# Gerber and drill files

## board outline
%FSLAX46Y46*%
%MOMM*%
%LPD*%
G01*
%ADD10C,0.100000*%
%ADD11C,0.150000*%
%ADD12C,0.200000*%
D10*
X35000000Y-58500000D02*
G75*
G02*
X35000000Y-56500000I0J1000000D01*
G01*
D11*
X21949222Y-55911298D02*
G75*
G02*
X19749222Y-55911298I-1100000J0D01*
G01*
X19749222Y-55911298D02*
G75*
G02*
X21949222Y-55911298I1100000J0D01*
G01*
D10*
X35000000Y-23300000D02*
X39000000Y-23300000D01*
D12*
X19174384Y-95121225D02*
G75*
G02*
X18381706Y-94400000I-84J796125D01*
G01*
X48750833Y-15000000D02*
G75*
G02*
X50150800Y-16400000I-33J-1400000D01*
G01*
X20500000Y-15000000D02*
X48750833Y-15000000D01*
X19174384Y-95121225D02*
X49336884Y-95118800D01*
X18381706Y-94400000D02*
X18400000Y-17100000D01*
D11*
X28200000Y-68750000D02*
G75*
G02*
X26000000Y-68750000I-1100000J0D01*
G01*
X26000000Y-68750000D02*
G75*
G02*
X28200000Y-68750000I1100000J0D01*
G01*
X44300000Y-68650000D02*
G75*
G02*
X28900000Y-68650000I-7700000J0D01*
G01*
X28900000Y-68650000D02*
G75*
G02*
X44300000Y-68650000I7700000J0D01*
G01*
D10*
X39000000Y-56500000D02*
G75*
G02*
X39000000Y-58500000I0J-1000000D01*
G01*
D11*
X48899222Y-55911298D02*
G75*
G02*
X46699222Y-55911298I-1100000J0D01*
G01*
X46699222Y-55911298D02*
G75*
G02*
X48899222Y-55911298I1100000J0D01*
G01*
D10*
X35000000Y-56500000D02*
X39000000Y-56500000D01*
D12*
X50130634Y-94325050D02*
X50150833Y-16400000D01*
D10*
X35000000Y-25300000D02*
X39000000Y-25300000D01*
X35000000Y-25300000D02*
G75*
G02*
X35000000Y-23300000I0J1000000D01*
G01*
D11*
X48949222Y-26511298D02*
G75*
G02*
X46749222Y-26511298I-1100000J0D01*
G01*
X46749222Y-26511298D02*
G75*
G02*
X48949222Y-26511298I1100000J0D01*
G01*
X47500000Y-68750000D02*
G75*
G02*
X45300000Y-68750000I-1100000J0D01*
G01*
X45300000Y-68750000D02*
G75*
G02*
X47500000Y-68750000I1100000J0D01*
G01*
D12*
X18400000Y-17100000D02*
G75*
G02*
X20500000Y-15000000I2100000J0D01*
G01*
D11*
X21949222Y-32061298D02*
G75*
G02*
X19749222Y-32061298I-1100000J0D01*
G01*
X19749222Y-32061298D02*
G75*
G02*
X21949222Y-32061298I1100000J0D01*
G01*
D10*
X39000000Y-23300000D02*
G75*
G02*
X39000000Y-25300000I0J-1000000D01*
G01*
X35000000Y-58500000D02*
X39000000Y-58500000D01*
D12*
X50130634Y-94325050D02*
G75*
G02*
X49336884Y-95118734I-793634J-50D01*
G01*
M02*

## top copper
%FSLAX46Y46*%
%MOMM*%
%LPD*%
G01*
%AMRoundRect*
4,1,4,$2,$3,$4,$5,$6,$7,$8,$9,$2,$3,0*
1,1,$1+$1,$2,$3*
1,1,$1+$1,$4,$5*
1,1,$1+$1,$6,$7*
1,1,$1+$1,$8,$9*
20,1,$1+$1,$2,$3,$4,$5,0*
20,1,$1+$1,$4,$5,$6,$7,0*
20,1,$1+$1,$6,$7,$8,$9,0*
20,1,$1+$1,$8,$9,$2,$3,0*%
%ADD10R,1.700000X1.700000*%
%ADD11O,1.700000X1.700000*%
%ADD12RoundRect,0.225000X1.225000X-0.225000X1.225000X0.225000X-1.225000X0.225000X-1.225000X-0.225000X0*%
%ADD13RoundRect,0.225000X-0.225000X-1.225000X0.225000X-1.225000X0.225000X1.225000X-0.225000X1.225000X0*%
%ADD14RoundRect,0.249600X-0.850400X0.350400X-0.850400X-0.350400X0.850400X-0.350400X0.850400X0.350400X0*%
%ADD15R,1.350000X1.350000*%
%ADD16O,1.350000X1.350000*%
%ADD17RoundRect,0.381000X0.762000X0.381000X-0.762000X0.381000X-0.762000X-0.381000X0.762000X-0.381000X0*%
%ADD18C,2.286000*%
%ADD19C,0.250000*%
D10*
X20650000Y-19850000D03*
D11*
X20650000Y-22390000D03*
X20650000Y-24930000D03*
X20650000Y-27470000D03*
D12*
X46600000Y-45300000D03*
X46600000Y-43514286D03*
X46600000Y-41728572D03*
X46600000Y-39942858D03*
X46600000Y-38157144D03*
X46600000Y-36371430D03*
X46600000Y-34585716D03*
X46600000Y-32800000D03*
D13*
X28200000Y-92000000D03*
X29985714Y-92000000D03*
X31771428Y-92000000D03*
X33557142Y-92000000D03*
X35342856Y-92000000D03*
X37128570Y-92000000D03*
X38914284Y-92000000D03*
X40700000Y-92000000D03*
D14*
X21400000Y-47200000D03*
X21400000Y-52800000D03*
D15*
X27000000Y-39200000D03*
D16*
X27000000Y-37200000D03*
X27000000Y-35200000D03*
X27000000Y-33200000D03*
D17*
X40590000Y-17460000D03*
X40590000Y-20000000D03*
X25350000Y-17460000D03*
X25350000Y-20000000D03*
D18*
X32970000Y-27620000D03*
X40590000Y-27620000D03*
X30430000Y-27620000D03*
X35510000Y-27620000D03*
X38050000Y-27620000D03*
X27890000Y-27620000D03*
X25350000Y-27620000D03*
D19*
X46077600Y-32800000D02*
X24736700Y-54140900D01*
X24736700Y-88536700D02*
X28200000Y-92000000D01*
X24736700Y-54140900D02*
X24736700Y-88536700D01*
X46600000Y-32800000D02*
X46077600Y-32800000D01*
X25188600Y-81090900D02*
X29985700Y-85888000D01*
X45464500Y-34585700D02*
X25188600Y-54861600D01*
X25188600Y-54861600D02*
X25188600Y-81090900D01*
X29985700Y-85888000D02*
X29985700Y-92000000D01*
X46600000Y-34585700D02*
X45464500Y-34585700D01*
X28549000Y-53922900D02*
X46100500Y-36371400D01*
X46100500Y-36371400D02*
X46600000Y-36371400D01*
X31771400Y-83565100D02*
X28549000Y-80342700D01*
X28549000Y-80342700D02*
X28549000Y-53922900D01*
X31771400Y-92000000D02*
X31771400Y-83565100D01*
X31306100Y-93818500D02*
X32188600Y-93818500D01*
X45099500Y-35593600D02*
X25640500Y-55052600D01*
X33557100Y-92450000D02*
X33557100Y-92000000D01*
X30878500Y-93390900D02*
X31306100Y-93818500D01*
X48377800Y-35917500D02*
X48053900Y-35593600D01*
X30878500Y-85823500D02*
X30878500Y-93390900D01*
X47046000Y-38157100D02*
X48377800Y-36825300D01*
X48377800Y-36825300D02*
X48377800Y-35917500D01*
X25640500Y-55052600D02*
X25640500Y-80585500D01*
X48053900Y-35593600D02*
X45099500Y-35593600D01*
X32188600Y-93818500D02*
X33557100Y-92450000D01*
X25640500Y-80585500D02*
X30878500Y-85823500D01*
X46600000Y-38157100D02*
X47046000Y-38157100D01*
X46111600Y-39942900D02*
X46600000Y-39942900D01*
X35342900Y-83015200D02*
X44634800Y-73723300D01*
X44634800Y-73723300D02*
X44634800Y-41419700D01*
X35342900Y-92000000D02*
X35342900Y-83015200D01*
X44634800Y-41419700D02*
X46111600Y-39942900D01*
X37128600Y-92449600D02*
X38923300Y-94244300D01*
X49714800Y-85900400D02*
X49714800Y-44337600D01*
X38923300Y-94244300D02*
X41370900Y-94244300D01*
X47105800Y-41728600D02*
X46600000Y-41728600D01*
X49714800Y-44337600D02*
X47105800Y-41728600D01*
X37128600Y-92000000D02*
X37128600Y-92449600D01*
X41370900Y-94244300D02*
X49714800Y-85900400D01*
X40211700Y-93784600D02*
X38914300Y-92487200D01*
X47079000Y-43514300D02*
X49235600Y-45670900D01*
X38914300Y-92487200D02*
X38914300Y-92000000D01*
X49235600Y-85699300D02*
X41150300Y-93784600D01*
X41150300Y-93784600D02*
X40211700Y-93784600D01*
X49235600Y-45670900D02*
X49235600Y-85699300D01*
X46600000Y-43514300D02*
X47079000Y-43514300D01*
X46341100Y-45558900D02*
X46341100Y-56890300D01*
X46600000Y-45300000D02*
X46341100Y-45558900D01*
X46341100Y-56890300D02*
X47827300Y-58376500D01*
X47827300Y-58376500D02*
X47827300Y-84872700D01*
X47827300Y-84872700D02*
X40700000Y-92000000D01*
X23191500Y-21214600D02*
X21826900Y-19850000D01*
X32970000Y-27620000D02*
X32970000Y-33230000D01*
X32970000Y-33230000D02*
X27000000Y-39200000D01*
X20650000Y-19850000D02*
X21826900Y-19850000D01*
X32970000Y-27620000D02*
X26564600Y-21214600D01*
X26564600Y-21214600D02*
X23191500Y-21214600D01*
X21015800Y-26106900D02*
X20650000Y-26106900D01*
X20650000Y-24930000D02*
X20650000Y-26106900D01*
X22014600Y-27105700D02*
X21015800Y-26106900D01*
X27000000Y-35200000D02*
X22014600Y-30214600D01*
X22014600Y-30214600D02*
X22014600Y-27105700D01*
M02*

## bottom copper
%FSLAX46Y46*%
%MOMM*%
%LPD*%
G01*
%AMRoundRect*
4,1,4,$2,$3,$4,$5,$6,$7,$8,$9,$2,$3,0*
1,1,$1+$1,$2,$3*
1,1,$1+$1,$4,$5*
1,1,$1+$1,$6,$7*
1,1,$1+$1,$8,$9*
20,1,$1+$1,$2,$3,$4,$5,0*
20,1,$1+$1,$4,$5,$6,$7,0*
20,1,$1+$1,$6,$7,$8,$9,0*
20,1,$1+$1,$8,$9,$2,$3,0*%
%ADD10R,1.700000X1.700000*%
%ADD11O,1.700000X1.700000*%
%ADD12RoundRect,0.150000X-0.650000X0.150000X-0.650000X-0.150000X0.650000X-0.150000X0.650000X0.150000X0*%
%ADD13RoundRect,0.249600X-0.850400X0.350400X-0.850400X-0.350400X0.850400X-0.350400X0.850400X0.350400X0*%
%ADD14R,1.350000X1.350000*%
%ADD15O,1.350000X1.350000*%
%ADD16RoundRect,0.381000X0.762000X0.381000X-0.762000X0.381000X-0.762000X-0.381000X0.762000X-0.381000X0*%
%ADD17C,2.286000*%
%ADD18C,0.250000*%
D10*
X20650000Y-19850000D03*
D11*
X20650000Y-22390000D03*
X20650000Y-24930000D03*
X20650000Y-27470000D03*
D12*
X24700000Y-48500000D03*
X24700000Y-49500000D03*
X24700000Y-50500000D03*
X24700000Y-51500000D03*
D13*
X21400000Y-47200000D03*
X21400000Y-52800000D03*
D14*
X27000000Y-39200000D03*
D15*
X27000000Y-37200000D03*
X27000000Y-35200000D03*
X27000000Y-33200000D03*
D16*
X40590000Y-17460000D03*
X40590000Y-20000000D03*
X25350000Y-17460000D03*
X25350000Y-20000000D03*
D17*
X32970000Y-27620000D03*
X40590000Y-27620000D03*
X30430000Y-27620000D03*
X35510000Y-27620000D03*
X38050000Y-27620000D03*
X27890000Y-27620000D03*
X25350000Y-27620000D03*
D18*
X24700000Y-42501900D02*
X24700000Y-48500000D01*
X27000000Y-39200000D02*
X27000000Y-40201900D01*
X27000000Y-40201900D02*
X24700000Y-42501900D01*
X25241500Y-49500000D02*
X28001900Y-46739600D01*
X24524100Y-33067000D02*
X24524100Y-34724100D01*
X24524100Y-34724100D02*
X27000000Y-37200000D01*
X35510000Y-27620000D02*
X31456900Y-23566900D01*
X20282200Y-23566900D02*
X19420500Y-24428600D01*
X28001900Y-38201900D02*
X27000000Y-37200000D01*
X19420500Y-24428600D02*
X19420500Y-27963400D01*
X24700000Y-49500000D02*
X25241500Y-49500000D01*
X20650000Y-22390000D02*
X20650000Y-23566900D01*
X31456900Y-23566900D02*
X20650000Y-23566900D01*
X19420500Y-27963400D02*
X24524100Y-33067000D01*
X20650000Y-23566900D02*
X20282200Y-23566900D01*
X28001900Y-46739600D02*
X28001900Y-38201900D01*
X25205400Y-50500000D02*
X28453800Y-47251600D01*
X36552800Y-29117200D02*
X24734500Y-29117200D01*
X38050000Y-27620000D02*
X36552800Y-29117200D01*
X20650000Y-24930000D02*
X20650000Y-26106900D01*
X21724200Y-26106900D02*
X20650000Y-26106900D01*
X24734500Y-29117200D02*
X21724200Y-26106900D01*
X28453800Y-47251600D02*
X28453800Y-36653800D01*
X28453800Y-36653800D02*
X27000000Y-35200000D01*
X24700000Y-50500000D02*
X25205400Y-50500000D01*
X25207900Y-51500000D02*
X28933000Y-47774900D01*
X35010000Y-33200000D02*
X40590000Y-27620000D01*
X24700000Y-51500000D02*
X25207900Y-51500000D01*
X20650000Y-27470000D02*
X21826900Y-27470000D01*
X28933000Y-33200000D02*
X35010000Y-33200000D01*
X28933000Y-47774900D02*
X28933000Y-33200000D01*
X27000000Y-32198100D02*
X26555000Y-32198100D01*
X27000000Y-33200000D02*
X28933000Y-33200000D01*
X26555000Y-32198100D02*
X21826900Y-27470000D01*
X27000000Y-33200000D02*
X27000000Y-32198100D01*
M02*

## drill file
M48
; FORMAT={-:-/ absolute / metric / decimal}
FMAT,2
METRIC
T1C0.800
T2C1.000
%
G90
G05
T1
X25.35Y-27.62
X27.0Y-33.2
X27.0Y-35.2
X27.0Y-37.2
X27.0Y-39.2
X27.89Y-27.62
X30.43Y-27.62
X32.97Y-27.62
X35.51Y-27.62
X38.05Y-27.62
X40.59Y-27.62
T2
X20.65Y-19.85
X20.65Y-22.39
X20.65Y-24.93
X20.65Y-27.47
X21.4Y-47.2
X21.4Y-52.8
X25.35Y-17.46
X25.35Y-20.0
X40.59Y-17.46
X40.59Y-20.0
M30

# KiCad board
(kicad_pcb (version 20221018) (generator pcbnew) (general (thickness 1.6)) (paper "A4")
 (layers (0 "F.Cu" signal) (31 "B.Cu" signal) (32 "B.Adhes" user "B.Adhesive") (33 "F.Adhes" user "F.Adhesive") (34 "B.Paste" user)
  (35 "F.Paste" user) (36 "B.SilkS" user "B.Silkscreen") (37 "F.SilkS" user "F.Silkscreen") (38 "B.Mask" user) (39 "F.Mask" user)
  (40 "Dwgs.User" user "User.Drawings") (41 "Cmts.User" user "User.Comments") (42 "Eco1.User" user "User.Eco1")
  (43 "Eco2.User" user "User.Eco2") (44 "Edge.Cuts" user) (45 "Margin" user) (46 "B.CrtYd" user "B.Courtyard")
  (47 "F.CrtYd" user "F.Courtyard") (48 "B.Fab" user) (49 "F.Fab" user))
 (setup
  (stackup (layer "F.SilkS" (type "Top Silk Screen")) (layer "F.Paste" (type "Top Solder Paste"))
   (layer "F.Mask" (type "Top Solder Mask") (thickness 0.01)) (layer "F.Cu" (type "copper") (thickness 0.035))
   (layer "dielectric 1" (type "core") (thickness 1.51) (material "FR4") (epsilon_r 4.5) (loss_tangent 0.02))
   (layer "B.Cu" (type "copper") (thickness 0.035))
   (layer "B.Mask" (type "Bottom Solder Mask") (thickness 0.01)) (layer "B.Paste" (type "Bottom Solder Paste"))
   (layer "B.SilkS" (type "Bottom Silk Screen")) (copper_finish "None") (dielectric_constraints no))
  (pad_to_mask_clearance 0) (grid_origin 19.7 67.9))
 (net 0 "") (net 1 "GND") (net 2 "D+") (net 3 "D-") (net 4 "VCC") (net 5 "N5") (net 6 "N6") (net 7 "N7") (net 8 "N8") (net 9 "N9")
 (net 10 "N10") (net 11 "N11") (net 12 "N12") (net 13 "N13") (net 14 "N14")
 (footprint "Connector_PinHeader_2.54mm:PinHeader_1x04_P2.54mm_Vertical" (layer "F.Cu") (at 20.65 19.85)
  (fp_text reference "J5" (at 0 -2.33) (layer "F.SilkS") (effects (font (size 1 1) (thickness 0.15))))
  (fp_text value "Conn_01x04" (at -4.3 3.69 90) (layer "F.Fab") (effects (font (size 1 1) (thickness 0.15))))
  (pad "1" thru_hole rect (at 0 0) (size 1.7 1.7) (drill 1) (layers "*.Cu" "*.Mask") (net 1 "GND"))
  (pad "2" thru_hole oval (at 0 2.54) (size 1.7 1.7) (drill 1) (layers "*.Cu" "*.Mask") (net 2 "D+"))
  (pad "3" thru_hole oval (at 0 5.08) (size 1.7 1.7) (drill 1) (layers "*.Cu" "*.Mask") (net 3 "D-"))
  (pad "4" thru_hole oval (at 0 7.62) (size 1.7 1.7) (drill 1) (layers "*.Cu" "*.Mask") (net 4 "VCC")))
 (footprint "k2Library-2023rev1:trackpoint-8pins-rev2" (layer "F.Cu") (at 44.1 38.55 90)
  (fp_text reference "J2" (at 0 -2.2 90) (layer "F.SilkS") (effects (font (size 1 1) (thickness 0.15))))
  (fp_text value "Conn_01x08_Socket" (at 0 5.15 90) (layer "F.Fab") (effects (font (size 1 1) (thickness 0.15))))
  (pad "1" smd roundrect (at -6.75 2.5 90) (size 0.9 2.9) (layers "F.Cu" "F.Paste" "F.Mask") (roundrect_rratio 0.25) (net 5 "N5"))
  (pad "2" smd roundrect (at -4.964286 2.5 90) (size 0.9 2.9) (layers "F.Cu" "F.Paste" "F.Mask") (roundrect_rratio 0.25) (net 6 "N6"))
  (pad "3" smd roundrect (at -3.178572 2.5 90) (size 0.9 2.9) (layers "F.Cu" "F.Paste" "F.Mask") (roundrect_rratio 0.25) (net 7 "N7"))
  (pad "4" smd roundrect (at -1.392858 2.5 90) (size 0.9 2.9) (layers "F.Cu" "F.Paste" "F.Mask") (roundrect_rratio 0.25) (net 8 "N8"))
  (pad "5" smd roundrect (at 0.392856 2.5 90) (size 0.9 2.9) (layers "F.Cu" "F.Paste" "F.Mask") (roundrect_rratio 0.25) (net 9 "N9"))
  (pad "6" smd roundrect (at 2.17857 2.5 90) (size 0.9 2.9) (layers "F.Cu" "F.Paste" "F.Mask") (roundrect_rratio 0.25) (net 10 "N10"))
  (pad "7" smd roundrect (at 3.964284 2.5 90) (size 0.9 2.9) (layers "F.Cu" "F.Paste" "F.Mask") (roundrect_rratio 0.25) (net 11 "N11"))
  (pad "8" smd roundrect (at 5.75 2.5 90) (size 0.9 2.9) (layers "F.Cu" "F.Paste" "F.Mask") (roundrect_rratio 0.25) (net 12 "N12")))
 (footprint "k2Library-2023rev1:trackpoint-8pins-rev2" (layer "F.Cu") (at 34.95 89.5)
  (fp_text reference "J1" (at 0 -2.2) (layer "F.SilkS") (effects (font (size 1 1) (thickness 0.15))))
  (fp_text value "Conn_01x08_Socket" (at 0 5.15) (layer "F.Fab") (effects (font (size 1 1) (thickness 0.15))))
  (pad "1" smd roundrect (at -6.75 2.5) (size 0.9 2.9) (layers "F.Cu" "F.Paste" "F.Mask") (roundrect_rratio 0.25) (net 12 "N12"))
  (pad "2" smd roundrect (at -4.964286 2.5) (size 0.9 2.9) (layers "F.Cu" "F.Paste" "F.Mask") (roundrect_rratio 0.25) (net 11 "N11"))
  (pad "3" smd roundrect (at -3.178572 2.5) (size 0.9 2.9) (layers "F.Cu" "F.Paste" "F.Mask") (roundrect_rratio 0.25) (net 10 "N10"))
  (pad "4" smd roundrect (at -1.392858 2.5) (size 0.9 2.9) (layers "F.Cu" "F.Paste" "F.Mask") (roundrect_rratio 0.25) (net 9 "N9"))
  (pad "5" smd roundrect (at 0.392856 2.5) (size 0.9 2.9) (layers "F.Cu" "F.Paste" "F.Mask") (roundrect_rratio 0.25) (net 8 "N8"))
  (pad "6" smd roundrect (at 2.17857 2.5) (size 0.9 2.9) (layers "F.Cu" "F.Paste" "F.Mask") (roundrect_rratio 0.25) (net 7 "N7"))
  (pad "7" smd roundrect (at 3.964284 2.5) (size 0.9 2.9) (layers "F.Cu" "F.Paste" "F.Mask") (roundrect_rratio 0.25) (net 6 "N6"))
  (pad "8" smd roundrect (at 5.75 2.5) (size 0.9 2.9) (layers "F.Cu" "F.Paste" "F.Mask") (roundrect_rratio 0.25) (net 5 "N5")))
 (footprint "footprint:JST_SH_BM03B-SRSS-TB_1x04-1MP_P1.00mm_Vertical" (layer "B.Cu") (at 22.9 50 -90)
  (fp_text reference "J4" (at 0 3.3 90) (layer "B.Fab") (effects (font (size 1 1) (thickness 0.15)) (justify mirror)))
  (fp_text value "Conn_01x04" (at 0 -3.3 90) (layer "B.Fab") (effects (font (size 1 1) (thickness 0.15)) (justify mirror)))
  (pad "1" smd roundrect (at -1.5 -1.8 270) (size 0.6 1.6) (layers "B.Cu" "B.Paste" "B.Mask") (roundrect_rratio 0.25) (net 1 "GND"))
  (pad "2" smd roundrect (at -0.5 -1.8 270) (size 0.6 1.6) (layers "B.Cu" "B.Paste" "B.Mask") (roundrect_rratio 0.25) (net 2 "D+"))
  (pad "3" smd roundrect (at 0.5 -1.8 270) (size 0.6 1.6) (layers "B.Cu" "B.Paste" "B.Mask") (roundrect_rratio 0.25) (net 3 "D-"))
  (pad "4" smd roundrect (at 1.5 -1.8 270) (size 0.6 1.6) (layers "B.Cu" "B.Paste" "B.Mask") (roundrect_rratio 0.25) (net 4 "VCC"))
  (pad "MP" thru_hole roundrect (at -2.8 1.5 270) (size 1.2 2.2) (drill 1) (layers "*.Cu" "*.Mask") (roundrect_rratio 0.208))
  (pad "MP" thru_hole roundrect (at 2.8 1.5 270) (size 1.2 2.2) (drill 1) (layers "*.Cu" "*.Mask") (roundrect_rratio 0.208)))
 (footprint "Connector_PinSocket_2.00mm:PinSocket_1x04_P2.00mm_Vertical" (layer "B.Cu") (at 27 39.2)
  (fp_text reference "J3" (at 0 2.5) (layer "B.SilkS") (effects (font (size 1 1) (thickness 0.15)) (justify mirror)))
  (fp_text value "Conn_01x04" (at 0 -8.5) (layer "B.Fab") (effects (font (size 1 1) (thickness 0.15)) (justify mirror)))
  (pad "1" thru_hole rect (at 0 0) (size 1.35 1.35) (drill 0.8) (layers "*.Cu" "*.Mask") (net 1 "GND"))
  (pad "2" thru_hole oval (at 0 -2) (size 1.35 1.35) (drill 0.8) (layers "*.Cu" "*.Mask") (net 2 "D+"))
  (pad "3" thru_hole oval (at 0 -4) (size 1.35 1.35) (drill 0.8) (layers "*.Cu" "*.Mask") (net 3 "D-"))
  (pad "4" thru_hole oval (at 0 -6) (size 1.35 1.35) (drill 0.8) (layers "*.Cu" "*.Mask") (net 4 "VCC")))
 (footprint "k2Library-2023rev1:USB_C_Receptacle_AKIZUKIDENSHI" (layer "B.Cu") (at 32.97 22.8 180)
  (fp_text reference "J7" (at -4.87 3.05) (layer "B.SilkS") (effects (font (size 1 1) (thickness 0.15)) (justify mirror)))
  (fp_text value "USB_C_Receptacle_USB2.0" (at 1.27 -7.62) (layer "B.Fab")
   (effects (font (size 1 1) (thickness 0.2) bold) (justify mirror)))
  (pad "1" thru_hole roundrect (at -7.62 5.34 180) (size 2.286 1.524) (drill 1) (layers "*.Cu" "*.Mask") (roundrect_rratio 0.25)
   (thermal_bridge_angle 45))
  (pad "2" thru_hole roundrect (at -7.62 2.8 180) (size 2.286 1.524) (drill 1) (layers "*.Cu" "*.Mask") (roundrect_rratio 0.25)
   (thermal_bridge_angle 45))
  (pad "3" thru_hole roundrect (at 7.62 5.34 180) (size 2.286 1.524) (drill 1) (layers "*.Cu" "*.Mask") (roundrect_rratio 0.25)
   (thermal_bridge_angle 45))
  (pad "4" thru_hole roundrect (at 7.62 2.8 180) (size 2.286 1.524) (drill 1) (layers "*.Cu" "*.Mask") (roundrect_rratio 0.25)
   (thermal_bridge_angle 45))
  (pad "A1" thru_hole circle (at 0 -4.82 90) (size 2.286 2.286) (drill 0.8) (layers "*.Cu" "*.Mask") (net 1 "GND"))
  (pad "A4" thru_hole circle (at -7.62 -4.82 180) (size 2.286 2.286) (drill 0.8) (layers "*.Cu" "*.Mask") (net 4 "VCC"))
  (pad "A5" thru_hole circle (at 2.54 -4.82 180) (size 2.286 2.286) (drill 0.8) (layers "*.Cu" "*.Mask") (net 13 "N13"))
  (pad "A6" thru_hole circle (at -2.54 -4.82 180) (size 2.286 2.286) (drill 0.8) (layers "*.Cu" "*.Mask") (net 2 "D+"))
  (pad "A7" thru_hole circle (at -5.08 -4.82 180) (size 2.286 2.286) (drill 0.8) (layers "*.Cu" "*.Mask") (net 3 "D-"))
  (pad "B5" thru_hole circle (at 5.08 -4.82 180) (size 2.286 2.286) (drill 0.8) (layers "*.Cu" "*.Mask") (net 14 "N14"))
  (pad "GND" thru_hole circle (at 7.62 -4.82 180) (size 2.286 2.286) (drill 0.8) (layers "*.Cu" "*.Mask")))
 (gr_arc (start 35 58.5) (mid 34 57.5) (end 35 56.5) (stroke (width 0.1) (type default)) (layer "Edge.Cuts"))
 (gr_circle (center 20.849222 55.911298) (end 21.949222 55.911298) (stroke (width 0.15) (type default)) (fill none) (layer "Edge.Cuts"))
 (gr_line (start 35 23.3) (end 39 23.3) (stroke (width 0.1) (type default)) (layer "Edge.Cuts"))
 (gr_arc (start 19.174384 95.121225) (mid 18.638521 94.91396) (end 18.381706 94.4) (stroke (width 0.2) (type solid)) (layer "Edge.Cuts"))
 (gr_arc (start 48.750833 15) (mid 49.740782 15.410051) (end 50.150833 16.4) (stroke (width 0.2) (type default)) (layer "Edge.Cuts"))
 (gr_line (start 20.5 15) (end 48.750833 15) (stroke (width 0.2) (type solid)) (layer "Edge.Cuts"))
 (gr_line (start 19.174384 95.121225) (end 49.336884 95.1188) (stroke (width 0.2) (type solid)) (layer "Edge.Cuts"))
 (gr_line (start 18.381706 94.4) (end 18.4 17.1) (stroke (width 0.2) (type solid)) (layer "Edge.Cuts"))
 (gr_circle (center 27.1 68.75) (end 28.2 68.75) (stroke (width 0.15) (type solid)) (fill none) (layer "Edge.Cuts"))
 (gr_circle (center 36.6 68.65) (end 44.3 68.65) (stroke (width 0.15) (type solid)) (fill none) (layer "Edge.Cuts"))
 (gr_arc (start 39 56.5) (mid 40 57.5) (end 39 58.5) (stroke (width 0.1) (type default)) (layer "Edge.Cuts"))
 (gr_circle (center 47.799222 55.911298) (end 48.899222 55.911298) (stroke (width 0.15) (type default)) (fill none) (layer "Edge.Cuts"))
 (gr_line (start 35 56.5) (end 39 56.5) (stroke (width 0.1) (type default)) (layer "Edge.Cuts"))
 (gr_line (start 50.130634 94.32505) (end 50.150833 16.4) (stroke (width 0.2) (type solid)) (layer "Edge.Cuts"))
 (gr_line (start 35 25.3) (end 39 25.3) (stroke (width 0.1) (type default)) (layer "Edge.Cuts"))
 (gr_arc (start 35 25.3) (mid 34 24.3) (end 35 23.3) (stroke (width 0.1) (type default)) (layer "Edge.Cuts"))
 (gr_circle (center 47.849222 26.511298) (end 48.949222 26.511298) (stroke (width 0.15) (type default)) (fill none) (layer "Edge.Cuts"))
 (gr_circle (center 46.4 68.75) (end 47.5 68.75) (stroke (width 0.15) (type solid)) (fill none) (layer "Edge.Cuts"))
 (gr_arc (start 18.4 17.1) (mid 19.015076 15.615076) (end 20.5 15) (stroke (width 0.2) (type default)) (layer "Edge.Cuts"))
 (gr_circle (center 20.849222 32.061298) (end 21.949222 32.061298) (stroke (width 0.15) (type default)) (fill none) (layer "Edge.Cuts"))
 (gr_arc (start 39 23.3) (mid 40 24.3) (end 39 25.3) (stroke (width 0.1) (type default)) (layer "Edge.Cuts"))
 (gr_line (start 35 58.5) (end 39 58.5) (stroke (width 0.1) (type default)) (layer "Edge.Cuts"))
 (gr_arc (start 50.130634 94.32505) (mid 49.898174 94.88634) (end 49.336884 95.1188) (stroke (width 0.2) (type solid)) (layer "Edge.Cuts"))
 (segment (start 46.0776 32.8) (end 24.7367 54.1409) (width 0.25) (layer "F.Cu") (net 12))
 (segment (start 24.7367 88.5367) (end 28.2 92) (width 0.25) (layer "F.Cu") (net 12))
 (segment (start 24.7367 54.1409) (end 24.7367 88.5367) (width 0.25) (layer "F.Cu") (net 12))
 (segment (start 46.6 32.8) (end 46.0776 32.8) (width 0.25) (layer "F.Cu") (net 12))
 (segment (start 25.1886 81.0909) (end 29.9857 85.888) (width 0.25) (layer "F.Cu") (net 11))
 (segment (start 45.4645 34.5857) (end 25.1886 54.8616) (width 0.25) (layer "F.Cu") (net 11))
 (segment (start 25.1886 54.8616) (end 25.1886 81.0909) (width 0.25) (layer "F.Cu") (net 11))
 (segment (start 29.9857 85.888) (end 29.9857 92) (width 0.25) (layer "F.Cu") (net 11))
 (segment (start 46.6 34.5857) (end 45.4645 34.5857) (width 0.25) (layer "F.Cu") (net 11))
 (segment (start 28.549 53.9229) (end 46.1005 36.3714) (width 0.25) (layer "F.Cu") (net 10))
 (segment (start 46.1005 36.3714) (end 46.6 36.3714) (width 0.25) (layer "F.Cu") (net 10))
 (segment (start 31.7714 83.5651) (end 28.549 80.3427) (width 0.25) (layer "F.Cu") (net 10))
 (segment (start 28.549 80.3427) (end 28.549 53.9229) (width 0.25) (layer "F.Cu") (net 10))
 (segment (start 31.7714 92) (end 31.7714 83.5651) (width 0.25) (layer "F.Cu") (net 10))
 (segment (start 31.3061 93.8185) (end 32.1886 93.8185) (width 0.25) (layer "F.Cu") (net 9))
 (segment (start 45.0995 35.5936) (end 25.6405 55.0526) (width 0.25) (layer "F.Cu") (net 9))
 (segment (start 33.5571 92.45) (end 33.5571 92) (width 0.25) (layer "F.Cu") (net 9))
 (segment (start 30.8785 93.3909) (end 31.3061 93.8185) (width 0.25) (layer "F.Cu") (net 9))
 (segment (start 48.3778 35.9175) (end 48.0539 35.5936) (width 0.25) (layer "F.Cu") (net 9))
 (segment (start 30.8785 85.8235) (end 30.8785 93.3909) (width 0.25) (layer "F.Cu") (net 9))
 (segment (start 47.046 38.1571) (end 48.3778 36.8253) (width 0.25) (layer "F.Cu") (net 9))
 (segment (start 48.3778 36.8253) (end 48.3778 35.9175) (width 0.25) (layer "F.Cu") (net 9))
 (segment (start 25.6405 55.0526) (end 25.6405 80.5855) (width 0.25) (layer "F.Cu") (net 9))
 (segment (start 48.0539 35.5936) (end 45.0995 35.5936) (width 0.25) (layer "F.Cu") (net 9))
 (segment (start 32.1886 93.8185) (end 33.5571 92.45) (width 0.25) (layer "F.Cu") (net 9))
 (segment (start 25.6405 80.5855) (end 30.8785 85.8235) (width 0.25) (layer "F.Cu") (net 9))
 (segment (start 46.6 38.1571) (end 47.046 38.1571) (width 0.25) (layer "F.Cu") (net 9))
 (segment (start 46.1116 39.9429) (end 46.6 39.9429) (width 0.25) (layer "F.Cu") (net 8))
 (segment (start 35.3429 83.0152) (end 44.6348 73.7233) (width 0.25) (layer "F.Cu") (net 8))
 (segment (start 44.6348 73.7233) (end 44.6348 41.4197) (width 0.25) (layer "F.Cu") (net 8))
 (segment (start 35.3429 92) (end 35.3429 83.0152) (width 0.25) (layer "F.Cu") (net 8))
 (segment (start 44.6348 41.4197) (end 46.1116 39.9429) (width 0.25) (layer "F.Cu") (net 8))
 (segment (start 37.1286 92.4496) (end 38.9233 94.2443) (width 0.25) (layer "F.Cu") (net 7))
 (segment (start 49.7148 85.9004) (end 49.7148 44.3376) (width 0.25) (layer "F.Cu") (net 7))
 (segment (start 38.9233 94.2443) (end 41.3709 94.2443) (width 0.25) (layer "F.Cu") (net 7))
 (segment (start 47.1058 41.7286) (end 46.6 41.7286) (width 0.25) (layer "F.Cu") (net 7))
 (segment (start 49.7148 44.3376) (end 47.1058 41.7286) (width 0.25) (layer "F.Cu") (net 7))
 (segment (start 37.1286 92) (end 37.1286 92.4496) (width 0.25) (layer "F.Cu") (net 7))
 (segment (start 41.3709 94.2443) (end 49.7148 85.9004) (width 0.25) (layer "F.Cu") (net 7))
 (segment (start 40.2117 93.7846) (end 38.9143 92.4872) (width 0.25) (layer "F.Cu") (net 6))
 (segment (start 47.079 43.5143) (end 49.2356 45.6709) (width 0.25) (layer "F.Cu") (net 6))
 (segment (start 38.9143 92.4872) (end 38.9143 92) (width 0.25) (layer "F.Cu") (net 6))
 (segment (start 49.2356 85.6993) (end 41.1503 93.7846) (width 0.25) (layer "F.Cu") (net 6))
 (segment (start 41.1503 93.7846) (end 40.2117 93.7846) (width 0.25) (layer "F.Cu") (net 6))
 (segment (start 49.2356 45.6709) (end 49.2356 85.6993) (width 0.25) (layer "F.Cu") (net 6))
 (segment (start 46.6 43.5143) (end 47.079 43.5143) (width 0.25) (layer "F.Cu") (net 6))
 (segment (start 46.3411 45.5589) (end 46.3411 56.8903) (width 0.25) (layer "F.Cu") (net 5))
 (segment (start 46.6 45.3) (end 46.3411 45.5589) (width 0.25) (layer "F.Cu") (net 5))
 (segment (start 46.3411 56.8903) (end 47.8273 58.3765) (width 0.25) (layer "F.Cu") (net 5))
 (segment (start 47.8273 58.3765) (end 47.8273 84.8727) (width 0.25) (layer "F.Cu") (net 5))
 (segment (start 47.8273 84.8727) (end 40.7 92) (width 0.25) (layer "F.Cu") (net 5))
 (segment (start 23.1915 21.2146) (end 21.8269 19.85) (width 0.25) (layer "F.Cu") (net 1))
 (segment (start 32.97 27.62) (end 32.97 33.23) (width 0.25) (layer "F.Cu") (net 1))
 (segment (start 32.97 33.23) (end 27 39.2) (width 0.25) (layer "F.Cu") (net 1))
 (segment (start 20.65 19.85) (end 21.8269 19.85) (width 0.25) (layer "F.Cu") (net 1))
 (segment (start 32.97 27.62) (end 26.5646 21.2146) (width 0.25) (layer "F.Cu") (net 1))
 (segment (start 26.5646 21.2146) (end 23.1915 21.2146) (width 0.25) (layer "F.Cu") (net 1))
 (segment (start 24.7 42.5019) (end 24.7 48.5) (width 0.25) (layer "B.Cu") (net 1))
 (segment (start 27 39.2) (end 27 40.2019) (width 0.25) (layer "B.Cu") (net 1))
 (segment (start 27 40.2019) (end 24.7 42.5019) (width 0.25) (layer "B.Cu") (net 1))
 (segment (start 25.2415 49.5) (end 28.0019 46.7396) (width 0.25) (layer "B.Cu") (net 2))
 (segment (start 24.5241 33.067) (end 24.5241 34.7241) (width 0.25) (layer "B.Cu") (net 2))
 (segment (start 24.5241 34.7241) (end 27 37.2) (width 0.25) (layer "B.Cu") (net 2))
 (segment (start 35.51 27.62) (end 31.4569 23.5669) (width 0.25) (layer "B.Cu") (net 2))
 (segment (start 20.2822 23.5669) (end 19.4205 24.4286) (width 0.25) (layer "B.Cu") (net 2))
 (segment (start 28.0019 38.2019) (end 27 37.2) (width 0.25) (layer "B.Cu") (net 2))
 (segment (start 19.4205 24.4286) (end 19.4205 27.9634) (width 0.25) (layer "B.Cu") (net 2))
 (segment (start 24.7 49.5) (end 25.2415 49.5) (width 0.25) (layer "B.Cu") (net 2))
 (segment (start 20.65 22.39) (end 20.65 23.5669) (width 0.25) (layer "B.Cu") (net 2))
 (segment (start 31.4569 23.5669) (end 20.65 23.5669) (width 0.25) (layer "B.Cu") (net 2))
 (segment (start 19.4205 27.9634) (end 24.5241 33.067) (width 0.25) (layer "B.Cu") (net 2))
 (segment (start 20.65 23.5669) (end 20.2822 23.5669) (width 0.25) (layer "B.Cu") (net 2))
 (segment (start 28.0019 46.7396) (end 28.0019 38.2019) (width 0.25) (layer "B.Cu") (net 2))
 (segment (start 21.0158 26.1069) (end 20.65 26.1069) (width 0.25) (layer "F.Cu") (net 3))
 (segment (start 20.65 24.93) (end 20.65 26.1069) (width 0.25) (layer "F.Cu") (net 3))
 (segment (start 22.0146 27.1057) (end 21.0158 26.1069) (width 0.25) (layer "F.Cu") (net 3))
 (segment (start 27 35.2) (end 22.0146 30.2146) (width 0.25) (layer "F.Cu") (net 3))
 (segment (start 22.0146 30.2146) (end 22.0146 27.1057) (width 0.25) (layer "F.Cu") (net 3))
 (segment (start 25.2054 50.5) (end 28.4538 47.2516) (width 0.25) (layer "B.Cu") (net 3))
 (segment (start 36.5528 29.1172) (end 24.7345 29.1172) (width 0.25) (layer "B.Cu") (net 3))
 (segment (start 38.05 27.62) (end 36.5528 29.1172) (width 0.25) (layer "B.Cu") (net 3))
 (segment (start 20.65 24.93) (end 20.65 26.1069) (width 0.25) (layer "B.Cu") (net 3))
 (segment (start 21.7242 26.1069) (end 20.65 26.1069) (width 0.25) (layer "B.Cu") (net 3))
 (segment (start 24.7345 29.1172) (end 21.7242 26.1069) (width 0.25) (layer "B.Cu") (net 3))
 (segment (start 28.4538 47.2516) (end 28.4538 36.6538) (width 0.25) (layer "B.Cu") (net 3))
 (segment (start 28.4538 36.6538) (end 27 35.2) (width 0.25) (layer "B.Cu") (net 3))
 (segment (start 24.7 50.5) (end 25.2054 50.5) (width 0.25) (layer "B.Cu") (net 3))
 (segment (start 25.2079 51.5) (end 28.933 47.7749) (width 0.25) (layer "B.Cu") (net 4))
 (segment (start 35.01 33.2) (end 40.59 27.62) (width 0.25) (layer "B.Cu") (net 4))
 (segment (start 24.7 51.5) (end 25.2079 51.5) (width 0.25) (layer "B.Cu") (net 4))
 (segment (start 20.65 27.47) (end 21.8269 27.47) (width 0.25) (layer "B.Cu") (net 4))
 (segment (start 28.933 33.2) (end 35.01 33.2) (width 0.25) (layer "B.Cu") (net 4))
 (segment (start 28.933 47.7749) (end 28.933 33.2) (width 0.25) (layer "B.Cu") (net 4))
 (segment (start 27 32.1981) (end 26.555 32.1981) (width 0.25) (layer "B.Cu") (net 4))
 (segment (start 27 33.2) (end 28.933 33.2) (width 0.25) (layer "B.Cu") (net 4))
 (segment (start 26.555 32.1981) (end 21.8269 27.47) (width 0.25) (layer "B.Cu") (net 4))
 (segment (start 27 33.2) (end 27 32.1981) (width 0.25) (layer "B.Cu") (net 4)))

